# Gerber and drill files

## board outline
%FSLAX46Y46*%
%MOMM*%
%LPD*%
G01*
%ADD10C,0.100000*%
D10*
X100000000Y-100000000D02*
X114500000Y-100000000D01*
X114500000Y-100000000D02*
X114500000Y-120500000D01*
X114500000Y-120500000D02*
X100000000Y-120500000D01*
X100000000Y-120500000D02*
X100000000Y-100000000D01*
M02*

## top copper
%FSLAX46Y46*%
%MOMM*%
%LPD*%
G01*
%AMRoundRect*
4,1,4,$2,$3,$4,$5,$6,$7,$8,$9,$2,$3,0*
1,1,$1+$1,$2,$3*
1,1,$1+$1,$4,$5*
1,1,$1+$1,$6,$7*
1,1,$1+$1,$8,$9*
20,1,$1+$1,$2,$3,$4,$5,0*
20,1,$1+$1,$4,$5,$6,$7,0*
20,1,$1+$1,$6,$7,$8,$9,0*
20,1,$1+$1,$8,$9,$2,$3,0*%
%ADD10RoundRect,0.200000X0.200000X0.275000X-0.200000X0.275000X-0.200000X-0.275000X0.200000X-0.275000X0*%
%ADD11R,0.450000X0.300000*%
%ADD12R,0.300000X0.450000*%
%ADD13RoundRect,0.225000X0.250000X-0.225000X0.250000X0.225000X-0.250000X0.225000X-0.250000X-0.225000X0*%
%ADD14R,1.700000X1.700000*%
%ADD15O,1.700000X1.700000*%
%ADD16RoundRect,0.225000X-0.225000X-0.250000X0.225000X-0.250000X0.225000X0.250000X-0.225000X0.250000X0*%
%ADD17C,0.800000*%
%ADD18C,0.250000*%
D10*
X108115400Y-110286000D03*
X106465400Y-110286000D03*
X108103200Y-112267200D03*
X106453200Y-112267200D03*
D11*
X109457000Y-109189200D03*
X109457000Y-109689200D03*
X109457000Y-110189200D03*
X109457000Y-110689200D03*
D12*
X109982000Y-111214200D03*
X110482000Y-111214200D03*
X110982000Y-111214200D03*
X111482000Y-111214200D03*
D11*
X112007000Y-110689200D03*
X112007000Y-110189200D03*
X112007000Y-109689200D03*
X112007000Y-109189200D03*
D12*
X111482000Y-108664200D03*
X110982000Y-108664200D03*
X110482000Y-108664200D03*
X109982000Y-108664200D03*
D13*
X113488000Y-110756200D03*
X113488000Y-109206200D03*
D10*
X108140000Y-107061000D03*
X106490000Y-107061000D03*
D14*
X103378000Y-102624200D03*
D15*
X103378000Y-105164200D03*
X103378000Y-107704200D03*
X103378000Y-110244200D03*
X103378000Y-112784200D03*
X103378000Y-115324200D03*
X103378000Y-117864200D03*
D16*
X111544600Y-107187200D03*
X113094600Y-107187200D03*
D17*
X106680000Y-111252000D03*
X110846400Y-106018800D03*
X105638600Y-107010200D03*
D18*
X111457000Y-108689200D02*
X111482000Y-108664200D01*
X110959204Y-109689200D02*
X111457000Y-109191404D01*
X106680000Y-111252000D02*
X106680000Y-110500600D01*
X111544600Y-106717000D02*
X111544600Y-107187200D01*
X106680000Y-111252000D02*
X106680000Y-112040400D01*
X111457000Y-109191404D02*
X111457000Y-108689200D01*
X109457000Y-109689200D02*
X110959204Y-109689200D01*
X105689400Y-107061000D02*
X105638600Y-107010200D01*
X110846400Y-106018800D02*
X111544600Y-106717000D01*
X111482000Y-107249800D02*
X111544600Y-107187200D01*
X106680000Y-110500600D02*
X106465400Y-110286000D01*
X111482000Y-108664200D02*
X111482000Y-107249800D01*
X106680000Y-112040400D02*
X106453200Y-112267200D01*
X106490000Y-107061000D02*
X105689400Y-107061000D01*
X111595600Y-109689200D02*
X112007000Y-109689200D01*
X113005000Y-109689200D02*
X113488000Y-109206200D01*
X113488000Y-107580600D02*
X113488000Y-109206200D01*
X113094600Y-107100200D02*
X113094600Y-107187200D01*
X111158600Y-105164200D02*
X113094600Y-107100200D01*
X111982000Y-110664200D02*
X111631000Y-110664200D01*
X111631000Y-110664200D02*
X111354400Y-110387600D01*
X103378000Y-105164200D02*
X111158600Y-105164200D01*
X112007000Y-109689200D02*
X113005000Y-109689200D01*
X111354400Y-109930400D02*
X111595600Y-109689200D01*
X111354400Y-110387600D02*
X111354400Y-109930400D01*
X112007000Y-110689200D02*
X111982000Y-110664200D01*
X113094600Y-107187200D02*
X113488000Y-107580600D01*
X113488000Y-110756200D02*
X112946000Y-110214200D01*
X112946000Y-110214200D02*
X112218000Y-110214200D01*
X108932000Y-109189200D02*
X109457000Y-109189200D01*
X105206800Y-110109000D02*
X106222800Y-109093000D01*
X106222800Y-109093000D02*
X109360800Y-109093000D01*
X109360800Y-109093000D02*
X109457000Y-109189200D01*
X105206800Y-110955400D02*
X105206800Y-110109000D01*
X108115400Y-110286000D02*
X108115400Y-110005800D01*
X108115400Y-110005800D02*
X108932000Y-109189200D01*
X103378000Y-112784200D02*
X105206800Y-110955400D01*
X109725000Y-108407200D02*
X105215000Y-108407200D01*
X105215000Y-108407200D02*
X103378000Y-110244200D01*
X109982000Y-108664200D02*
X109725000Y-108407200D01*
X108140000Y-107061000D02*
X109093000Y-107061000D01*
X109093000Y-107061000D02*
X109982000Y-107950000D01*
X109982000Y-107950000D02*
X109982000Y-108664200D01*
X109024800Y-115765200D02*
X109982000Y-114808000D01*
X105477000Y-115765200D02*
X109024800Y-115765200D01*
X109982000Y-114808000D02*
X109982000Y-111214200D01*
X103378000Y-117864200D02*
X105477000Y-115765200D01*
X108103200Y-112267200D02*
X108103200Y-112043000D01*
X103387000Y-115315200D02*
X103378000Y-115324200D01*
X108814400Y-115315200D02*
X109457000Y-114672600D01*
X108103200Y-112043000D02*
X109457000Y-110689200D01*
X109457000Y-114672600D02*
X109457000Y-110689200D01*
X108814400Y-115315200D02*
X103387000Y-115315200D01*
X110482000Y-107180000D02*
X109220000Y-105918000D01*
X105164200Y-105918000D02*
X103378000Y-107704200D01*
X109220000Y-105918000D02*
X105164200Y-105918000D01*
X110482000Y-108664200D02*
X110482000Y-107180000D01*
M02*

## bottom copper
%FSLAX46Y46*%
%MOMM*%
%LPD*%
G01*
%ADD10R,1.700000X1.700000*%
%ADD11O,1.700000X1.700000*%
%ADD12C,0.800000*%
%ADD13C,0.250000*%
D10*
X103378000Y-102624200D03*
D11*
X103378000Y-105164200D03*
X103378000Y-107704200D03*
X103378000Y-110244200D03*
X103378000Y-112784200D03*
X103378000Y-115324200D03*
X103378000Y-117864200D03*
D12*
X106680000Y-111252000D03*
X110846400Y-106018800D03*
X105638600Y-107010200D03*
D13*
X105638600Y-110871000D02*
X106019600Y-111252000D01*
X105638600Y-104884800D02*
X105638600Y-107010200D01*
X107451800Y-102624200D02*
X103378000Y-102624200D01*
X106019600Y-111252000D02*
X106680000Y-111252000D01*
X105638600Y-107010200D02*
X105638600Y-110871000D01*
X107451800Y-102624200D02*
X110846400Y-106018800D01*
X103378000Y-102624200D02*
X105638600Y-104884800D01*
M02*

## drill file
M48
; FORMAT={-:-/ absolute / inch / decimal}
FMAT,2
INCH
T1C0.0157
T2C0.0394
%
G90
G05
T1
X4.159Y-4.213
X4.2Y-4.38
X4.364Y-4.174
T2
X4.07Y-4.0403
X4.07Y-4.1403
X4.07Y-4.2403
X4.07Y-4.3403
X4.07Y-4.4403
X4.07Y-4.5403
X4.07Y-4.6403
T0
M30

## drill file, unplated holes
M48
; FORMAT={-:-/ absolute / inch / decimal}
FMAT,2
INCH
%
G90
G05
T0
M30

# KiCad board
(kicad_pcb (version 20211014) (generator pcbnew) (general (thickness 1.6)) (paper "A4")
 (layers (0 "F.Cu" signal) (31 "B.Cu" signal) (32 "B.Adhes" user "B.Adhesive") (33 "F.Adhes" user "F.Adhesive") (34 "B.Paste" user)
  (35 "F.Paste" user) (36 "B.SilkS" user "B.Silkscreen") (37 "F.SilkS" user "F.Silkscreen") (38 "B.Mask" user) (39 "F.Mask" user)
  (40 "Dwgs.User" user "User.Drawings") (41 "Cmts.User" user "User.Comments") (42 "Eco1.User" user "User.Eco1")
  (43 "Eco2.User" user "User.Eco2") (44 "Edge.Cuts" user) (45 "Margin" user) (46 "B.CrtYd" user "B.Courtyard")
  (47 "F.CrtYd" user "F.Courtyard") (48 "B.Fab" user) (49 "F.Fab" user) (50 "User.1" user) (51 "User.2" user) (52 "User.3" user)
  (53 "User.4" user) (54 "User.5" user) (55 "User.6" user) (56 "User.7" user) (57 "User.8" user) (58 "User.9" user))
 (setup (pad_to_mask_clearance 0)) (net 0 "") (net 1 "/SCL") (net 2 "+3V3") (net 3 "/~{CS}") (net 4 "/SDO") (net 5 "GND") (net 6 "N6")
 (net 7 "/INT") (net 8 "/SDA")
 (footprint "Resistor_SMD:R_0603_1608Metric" (layer "F.Cu") (at 107.2904 110.286 180)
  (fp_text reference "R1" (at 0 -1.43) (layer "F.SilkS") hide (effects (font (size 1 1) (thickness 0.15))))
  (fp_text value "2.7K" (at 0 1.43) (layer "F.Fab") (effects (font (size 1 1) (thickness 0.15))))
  (pad "1" smd roundrect (at -0.825 0 180) (size 0.8 0.95) (layers "F.Cu" "F.Paste" "F.Mask") (roundrect_rratio 0.25) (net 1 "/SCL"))
  (pad "2" smd roundrect (at 0.825 0 180) (size 0.8 0.95) (layers "F.Cu" "F.Paste" "F.Mask") (roundrect_rratio 0.25) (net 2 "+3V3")))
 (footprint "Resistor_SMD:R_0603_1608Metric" (layer "F.Cu") (at 107.2782 112.2672 180)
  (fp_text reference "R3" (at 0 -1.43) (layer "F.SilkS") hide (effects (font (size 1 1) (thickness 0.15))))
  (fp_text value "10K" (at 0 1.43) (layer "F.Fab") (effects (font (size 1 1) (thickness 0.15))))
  (pad "1" smd roundrect (at -0.825 0 180) (size 0.8 0.95) (layers "F.Cu" "F.Paste" "F.Mask") (roundrect_rratio 0.25) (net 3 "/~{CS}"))
  (pad "2" smd roundrect (at 0.825 0 180) (size 0.8 0.95) (layers "F.Cu" "F.Paste" "F.Mask") (roundrect_rratio 0.25) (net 2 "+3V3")))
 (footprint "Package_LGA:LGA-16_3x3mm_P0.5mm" (layer "F.Cu") (at 110.732 109.9392)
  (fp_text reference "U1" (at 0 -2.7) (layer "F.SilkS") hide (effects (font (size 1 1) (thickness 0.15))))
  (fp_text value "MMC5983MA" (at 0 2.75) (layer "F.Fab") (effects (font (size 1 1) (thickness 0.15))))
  (pad "1" smd rect (at -1.275 -0.75 90) (size 0.3 0.45) (layers "F.Cu" "F.Paste" "F.Mask") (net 1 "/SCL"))
  (pad "2" smd rect (at -1.275 -0.25 90) (size 0.3 0.45) (layers "F.Cu" "F.Paste" "F.Mask") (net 2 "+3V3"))
  (pad "3" smd rect (at -1.275 0.25 90) (size 0.3 0.45) (layers "F.Cu" "F.Paste" "F.Mask"))
  (pad "4" smd rect (at -1.275 0.75 90) (size 0.3 0.45) (layers "F.Cu" "F.Paste" "F.Mask") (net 3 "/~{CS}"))
  (pad "5" smd rect (at -0.75 1.275) (size 0.3 0.45) (layers "F.Cu" "F.Paste" "F.Mask") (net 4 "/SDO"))
  (pad "6" smd rect (at -0.25 1.275) (size 0.3 0.45) (layers "F.Cu" "F.Paste" "F.Mask"))
  (pad "7" smd rect (at 0.25 1.275) (size 0.3 0.45) (layers "F.Cu" "F.Paste" "F.Mask"))
  (pad "8" smd rect (at 0.75 1.275) (size 0.3 0.45) (layers "F.Cu" "F.Paste" "F.Mask"))
  (pad "9" smd rect (at 1.275 0.75 90) (size 0.3 0.45) (layers "F.Cu" "F.Paste" "F.Mask") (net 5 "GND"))
  (pad "10" smd rect (at 1.275 0.25 90) (size 0.3 0.45) (layers "F.Cu" "F.Paste" "F.Mask") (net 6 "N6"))
  (pad "11" smd rect (at 1.275 -0.25 90) (size 0.3 0.45) (layers "F.Cu" "F.Paste" "F.Mask") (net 5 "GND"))
  (pad "12" smd rect (at 1.275 -0.75 90) (size 0.3 0.45) (layers "F.Cu" "F.Paste" "F.Mask"))
  (pad "13" smd rect (at 0.75 -1.275) (size 0.3 0.45) (layers "F.Cu" "F.Paste" "F.Mask") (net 2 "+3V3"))
  (pad "14" smd rect (at 0.25 -1.275) (size 0.3 0.45) (layers "F.Cu" "F.Paste" "F.Mask"))
  (pad "15" smd rect (at -0.25 -1.275) (size 0.3 0.45) (layers "F.Cu" "F.Paste" "F.Mask") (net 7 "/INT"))
  (pad "16" smd rect (at -0.75 -1.275) (size 0.3 0.45) (layers "F.Cu" "F.Paste" "F.Mask") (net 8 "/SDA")))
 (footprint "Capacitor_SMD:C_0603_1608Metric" (layer "F.Cu") (at 113.488 109.9812 90)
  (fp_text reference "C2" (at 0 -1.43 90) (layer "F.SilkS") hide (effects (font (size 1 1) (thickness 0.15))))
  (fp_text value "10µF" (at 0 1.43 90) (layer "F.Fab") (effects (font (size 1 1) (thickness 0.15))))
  (pad "1" smd roundrect (at -0.775 0 90) (size 0.9 0.95) (layers "F.Cu" "F.Paste" "F.Mask") (roundrect_rratio 0.25) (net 6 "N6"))
  (pad "2" smd roundrect (at 0.775 0 90) (size 0.9 0.95) (layers "F.Cu" "F.Paste" "F.Mask") (roundrect_rratio 0.25) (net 5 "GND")))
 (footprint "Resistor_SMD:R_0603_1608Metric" (layer "F.Cu") (at 107.315 107.061 180)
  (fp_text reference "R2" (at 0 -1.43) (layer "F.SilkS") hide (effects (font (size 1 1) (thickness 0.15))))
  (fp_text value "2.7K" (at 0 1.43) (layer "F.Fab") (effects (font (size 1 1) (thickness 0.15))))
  (pad "1" smd roundrect (at -0.825 0 180) (size 0.8 0.95) (layers "F.Cu" "F.Paste" "F.Mask") (roundrect_rratio 0.25) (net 8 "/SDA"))
  (pad "2" smd roundrect (at 0.825 0 180) (size 0.8 0.95) (layers "F.Cu" "F.Paste" "F.Mask") (roundrect_rratio 0.25) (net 2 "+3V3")))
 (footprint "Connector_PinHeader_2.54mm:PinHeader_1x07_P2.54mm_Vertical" (layer "F.Cu") (at 103.378 102.6242)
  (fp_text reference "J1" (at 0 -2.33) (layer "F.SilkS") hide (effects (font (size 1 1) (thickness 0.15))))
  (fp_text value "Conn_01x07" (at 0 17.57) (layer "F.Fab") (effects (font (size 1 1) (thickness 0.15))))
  (pad "1" thru_hole rect (at 0 0) (size 1.7 1.7) (drill 1) (layers *.Cu *.Mask) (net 2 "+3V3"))
  (pad "2" thru_hole oval (at 0 2.54) (size 1.7 1.7) (drill 1) (layers *.Cu *.Mask) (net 5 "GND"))
  (pad "3" thru_hole oval (at 0 5.08) (size 1.7 1.7) (drill 1) (layers *.Cu *.Mask) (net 7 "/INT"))
  (pad "4" thru_hole oval (at 0 7.62) (size 1.7 1.7) (drill 1) (layers *.Cu *.Mask) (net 8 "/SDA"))
  (pad "5" thru_hole oval (at 0 10.16) (size 1.7 1.7) (drill 1) (layers *.Cu *.Mask) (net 1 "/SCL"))
  (pad "6" thru_hole oval (at 0 12.7) (size 1.7 1.7) (drill 1) (layers *.Cu *.Mask) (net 3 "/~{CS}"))
  (pad "7" thru_hole oval (at 0 15.24) (size 1.7 1.7) (drill 1) (layers *.Cu *.Mask) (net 4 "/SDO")))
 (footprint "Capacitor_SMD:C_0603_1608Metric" (layer "F.Cu") (at 112.3196 107.1872)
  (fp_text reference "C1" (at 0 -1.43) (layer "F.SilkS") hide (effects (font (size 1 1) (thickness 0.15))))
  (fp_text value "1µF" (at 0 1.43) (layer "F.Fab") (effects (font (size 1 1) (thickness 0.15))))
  (pad "1" smd roundrect (at -0.775 0) (size 0.9 0.95) (layers "F.Cu" "F.Paste" "F.Mask") (roundrect_rratio 0.25) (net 2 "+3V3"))
  (pad "2" smd roundrect (at 0.775 0) (size 0.9 0.95) (layers "F.Cu" "F.Paste" "F.Mask") (roundrect_rratio 0.25) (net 5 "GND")))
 (gr_rect (start 100 100) (end 114.5 120.5) (layer "Edge.Cuts") (width 0.1) (fill none))
 (segment (start 111.457 108.6892) (end 111.482 108.6642) (width 0.25) (layer "F.Cu") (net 2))
 (segment (start 110.959204 109.6892) (end 111.457 109.191404) (width 0.25) (layer "F.Cu") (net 2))
 (segment (start 106.68 111.252) (end 106.68 110.5006) (width 0.25) (layer "F.Cu") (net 2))
 (segment (start 111.5446 106.717) (end 111.5446 107.1872) (width 0.25) (layer "F.Cu") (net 2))
 (segment (start 106.68 111.252) (end 106.68 112.0404) (width 0.25) (layer "F.Cu") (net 2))
 (segment (start 111.457 109.191404) (end 111.457 108.6892) (width 0.25) (layer "F.Cu") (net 2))
 (segment (start 109.457 109.6892) (end 110.959204 109.6892) (width 0.25) (layer "F.Cu") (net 2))
 (segment (start 105.6894 107.061) (end 105.6386 107.0102) (width 0.25) (layer "F.Cu") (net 2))
 (segment (start 110.8464 106.0188) (end 111.5446 106.717) (width 0.25) (layer "F.Cu") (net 2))
 (segment (start 111.482 107.2498) (end 111.5446 107.1872) (width 0.25) (layer "F.Cu") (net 2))
 (segment (start 106.68 110.5006) (end 106.4654 110.286) (width 0.25) (layer "F.Cu") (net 2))
 (segment (start 111.482 108.6642) (end 111.482 107.2498) (width 0.25) (layer "F.Cu") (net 2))
 (segment (start 106.68 112.0404) (end 106.4532 112.2672) (width 0.25) (layer "F.Cu") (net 2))
 (segment (start 106.49 107.061) (end 105.6894 107.061) (width 0.25) (layer "F.Cu") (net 2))
 (via (at 106.68 111.252) (size 0.8) (drill 0.4) (layers "F.Cu" "B.Cu") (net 2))
 (via (at 110.8464 106.0188) (size 0.8) (drill 0.4) (layers "F.Cu" "B.Cu") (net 2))
 (via (at 105.6386 107.0102) (size 0.8) (drill 0.4) (layers "F.Cu" "B.Cu") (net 2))
 (segment (start 105.6386 110.871) (end 106.0196 111.252) (width 0.25) (layer "B.Cu") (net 2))
 (segment (start 105.6386 104.8848) (end 105.6386 107.0102) (width 0.25) (layer "B.Cu") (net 2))
 (segment (start 107.4518 102.6242) (end 103.378 102.6242) (width 0.25) (layer "B.Cu") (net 2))
 (segment (start 106.0196 111.252) (end 106.68 111.252) (width 0.25) (layer "B.Cu") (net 2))
 (segment (start 105.6386 107.0102) (end 105.6386 110.871) (width 0.25) (layer "B.Cu") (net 2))
 (segment (start 107.4518 102.6242) (end 110.8464 106.0188) (width 0.25) (layer "B.Cu") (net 2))
 (segment (start 103.378 102.6242) (end 105.6386 104.8848) (width 0.25) (layer "B.Cu") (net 2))
 (segment (start 111.5956 109.6892) (end 112.007 109.6892) (width 0.25) (layer "F.Cu") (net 5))
 (segment (start 113.005 109.6892) (end 113.488 109.2062) (width 0.25) (layer "F.Cu") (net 5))
 (segment (start 113.488 107.5806) (end 113.488 109.2062) (width 0.25) (layer "F.Cu") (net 5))
 (segment (start 113.0946 107.1002) (end 113.0946 107.1872) (width 0.25) (layer "F.Cu") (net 5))
 (segment (start 111.1586 105.1642) (end 113.0946 107.1002) (width 0.25) (layer "F.Cu") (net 5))
 (segment (start 111.982 110.6642) (end 111.631 110.6642) (width 0.25) (layer "F.Cu") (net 5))
 (segment (start 111.631 110.6642) (end 111.3544 110.3876) (width 0.25) (layer "F.Cu") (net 5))
 (segment (start 103.378 105.1642) (end 111.1586 105.1642) (width 0.25) (layer "F.Cu") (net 5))
 (segment (start 112.007 109.6892) (end 113.005 109.6892) (width 0.25) (layer "F.Cu") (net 5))
 (segment (start 111.3544 109.9304) (end 111.5956 109.6892) (width 0.25) (layer "F.Cu") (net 5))
 (segment (start 111.3544 110.3876) (end 111.3544 109.9304) (width 0.25) (layer "F.Cu") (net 5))
 (segment (start 112.007 110.6892) (end 111.982 110.6642) (width 0.25) (layer "F.Cu") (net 5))
 (segment (start 113.0946 107.1872) (end 113.488 107.5806) (width 0.25) (layer "F.Cu") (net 5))
 (segment (start 113.488 110.7562) (end 112.946 110.2142) (width 0.25) (layer "F.Cu") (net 6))
 (segment (start 112.946 110.2142) (end 112.218 110.2142) (width 0.25) (layer "F.Cu") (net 6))
 (segment (start 108.932 109.1892) (end 109.457 109.1892) (width 0.25) (layer "F.Cu") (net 1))
 (segment (start 105.2068 110.109) (end 106.2228 109.093) (width 0.25) (layer "F.Cu") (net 1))
 (segment (start 106.2228 109.093) (end 109.3608 109.093) (width 0.25) (layer "F.Cu") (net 1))
 (segment (start 109.3608 109.093) (end 109.457 109.1892) (width 0.25) (layer "F.Cu") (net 1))
 (segment (start 105.2068 110.9554) (end 105.2068 110.109) (width 0.25) (layer "F.Cu") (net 1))
 (segment (start 108.1154 110.286) (end 108.1154 110.0058) (width 0.25) (layer "F.Cu") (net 1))
 (segment (start 108.1154 110.0058) (end 108.932 109.1892) (width 0.25) (layer "F.Cu") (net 1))
 (segment (start 103.378 112.7842) (end 105.2068 110.9554) (width 0.25) (layer "F.Cu") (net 1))
 (segment (start 109.725 108.4072) (end 105.215 108.4072) (width 0.25) (layer "F.Cu") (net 8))
 (segment (start 105.215 108.4072) (end 103.378 110.2442) (width 0.25) (layer "F.Cu") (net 8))
 (segment (start 109.982 108.6642) (end 109.725 108.4072) (width 0.25) (layer "F.Cu") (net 8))
 (segment (start 108.14 107.061) (end 109.093 107.061) (width 0.25) (layer "F.Cu") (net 8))
 (segment (start 109.093 107.061) (end 109.982 107.95) (width 0.25) (layer "F.Cu") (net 8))
 (segment (start 109.982 107.95) (end 109.982 108.6642) (width 0.25) (layer "F.Cu") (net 8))
 (segment (start 109.0248 115.7652) (end 109.982 114.808) (width 0.25) (layer "F.Cu") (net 4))
 (segment (start 105.477 115.7652) (end 109.0248 115.7652) (width 0.25) (layer "F.Cu") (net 4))
 (segment (start 109.982 114.808) (end 109.982 111.2142) (width 0.25) (layer "F.Cu") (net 4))
 (segment (start 103.378 117.8642) (end 105.477 115.7652) (width 0.25) (layer "F.Cu") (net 4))
 (segment (start 108.1032 112.2672) (end 108.1032 112.043) (width 0.25) (layer "F.Cu") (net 3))
 (segment (start 103.387 115.3152) (end 103.378 115.3242) (width 0.25) (layer "F.Cu") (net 3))
 (segment (start 108.8144 115.3152) (end 109.457 114.6726) (width 0.25) (layer "F.Cu") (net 3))
 (segment (start 108.1032 112.043) (end 109.457 110.6892) (width 0.25) (layer "F.Cu") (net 3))
 (segment (start 109.457 114.6726) (end 109.457 110.6892) (width 0.25) (layer "F.Cu") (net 3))
 (segment (start 108.8144 115.3152) (end 103.387 115.3152) (width 0.25) (layer "F.Cu") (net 3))
 (segment (start 110.482 107.18) (end 109.22 105.918) (width 0.25) (layer "F.Cu") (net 7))
 (segment (start 105.1642 105.918) (end 103.378 107.7042) (width 0.25) (layer "F.Cu") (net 7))
 (segment (start 109.22 105.918) (end 105.1642 105.918) (width 0.25) (layer "F.Cu") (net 7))
 (segment (start 110.482 108.6642) (end 110.482 107.18) (width 0.25) (layer "F.Cu") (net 7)))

